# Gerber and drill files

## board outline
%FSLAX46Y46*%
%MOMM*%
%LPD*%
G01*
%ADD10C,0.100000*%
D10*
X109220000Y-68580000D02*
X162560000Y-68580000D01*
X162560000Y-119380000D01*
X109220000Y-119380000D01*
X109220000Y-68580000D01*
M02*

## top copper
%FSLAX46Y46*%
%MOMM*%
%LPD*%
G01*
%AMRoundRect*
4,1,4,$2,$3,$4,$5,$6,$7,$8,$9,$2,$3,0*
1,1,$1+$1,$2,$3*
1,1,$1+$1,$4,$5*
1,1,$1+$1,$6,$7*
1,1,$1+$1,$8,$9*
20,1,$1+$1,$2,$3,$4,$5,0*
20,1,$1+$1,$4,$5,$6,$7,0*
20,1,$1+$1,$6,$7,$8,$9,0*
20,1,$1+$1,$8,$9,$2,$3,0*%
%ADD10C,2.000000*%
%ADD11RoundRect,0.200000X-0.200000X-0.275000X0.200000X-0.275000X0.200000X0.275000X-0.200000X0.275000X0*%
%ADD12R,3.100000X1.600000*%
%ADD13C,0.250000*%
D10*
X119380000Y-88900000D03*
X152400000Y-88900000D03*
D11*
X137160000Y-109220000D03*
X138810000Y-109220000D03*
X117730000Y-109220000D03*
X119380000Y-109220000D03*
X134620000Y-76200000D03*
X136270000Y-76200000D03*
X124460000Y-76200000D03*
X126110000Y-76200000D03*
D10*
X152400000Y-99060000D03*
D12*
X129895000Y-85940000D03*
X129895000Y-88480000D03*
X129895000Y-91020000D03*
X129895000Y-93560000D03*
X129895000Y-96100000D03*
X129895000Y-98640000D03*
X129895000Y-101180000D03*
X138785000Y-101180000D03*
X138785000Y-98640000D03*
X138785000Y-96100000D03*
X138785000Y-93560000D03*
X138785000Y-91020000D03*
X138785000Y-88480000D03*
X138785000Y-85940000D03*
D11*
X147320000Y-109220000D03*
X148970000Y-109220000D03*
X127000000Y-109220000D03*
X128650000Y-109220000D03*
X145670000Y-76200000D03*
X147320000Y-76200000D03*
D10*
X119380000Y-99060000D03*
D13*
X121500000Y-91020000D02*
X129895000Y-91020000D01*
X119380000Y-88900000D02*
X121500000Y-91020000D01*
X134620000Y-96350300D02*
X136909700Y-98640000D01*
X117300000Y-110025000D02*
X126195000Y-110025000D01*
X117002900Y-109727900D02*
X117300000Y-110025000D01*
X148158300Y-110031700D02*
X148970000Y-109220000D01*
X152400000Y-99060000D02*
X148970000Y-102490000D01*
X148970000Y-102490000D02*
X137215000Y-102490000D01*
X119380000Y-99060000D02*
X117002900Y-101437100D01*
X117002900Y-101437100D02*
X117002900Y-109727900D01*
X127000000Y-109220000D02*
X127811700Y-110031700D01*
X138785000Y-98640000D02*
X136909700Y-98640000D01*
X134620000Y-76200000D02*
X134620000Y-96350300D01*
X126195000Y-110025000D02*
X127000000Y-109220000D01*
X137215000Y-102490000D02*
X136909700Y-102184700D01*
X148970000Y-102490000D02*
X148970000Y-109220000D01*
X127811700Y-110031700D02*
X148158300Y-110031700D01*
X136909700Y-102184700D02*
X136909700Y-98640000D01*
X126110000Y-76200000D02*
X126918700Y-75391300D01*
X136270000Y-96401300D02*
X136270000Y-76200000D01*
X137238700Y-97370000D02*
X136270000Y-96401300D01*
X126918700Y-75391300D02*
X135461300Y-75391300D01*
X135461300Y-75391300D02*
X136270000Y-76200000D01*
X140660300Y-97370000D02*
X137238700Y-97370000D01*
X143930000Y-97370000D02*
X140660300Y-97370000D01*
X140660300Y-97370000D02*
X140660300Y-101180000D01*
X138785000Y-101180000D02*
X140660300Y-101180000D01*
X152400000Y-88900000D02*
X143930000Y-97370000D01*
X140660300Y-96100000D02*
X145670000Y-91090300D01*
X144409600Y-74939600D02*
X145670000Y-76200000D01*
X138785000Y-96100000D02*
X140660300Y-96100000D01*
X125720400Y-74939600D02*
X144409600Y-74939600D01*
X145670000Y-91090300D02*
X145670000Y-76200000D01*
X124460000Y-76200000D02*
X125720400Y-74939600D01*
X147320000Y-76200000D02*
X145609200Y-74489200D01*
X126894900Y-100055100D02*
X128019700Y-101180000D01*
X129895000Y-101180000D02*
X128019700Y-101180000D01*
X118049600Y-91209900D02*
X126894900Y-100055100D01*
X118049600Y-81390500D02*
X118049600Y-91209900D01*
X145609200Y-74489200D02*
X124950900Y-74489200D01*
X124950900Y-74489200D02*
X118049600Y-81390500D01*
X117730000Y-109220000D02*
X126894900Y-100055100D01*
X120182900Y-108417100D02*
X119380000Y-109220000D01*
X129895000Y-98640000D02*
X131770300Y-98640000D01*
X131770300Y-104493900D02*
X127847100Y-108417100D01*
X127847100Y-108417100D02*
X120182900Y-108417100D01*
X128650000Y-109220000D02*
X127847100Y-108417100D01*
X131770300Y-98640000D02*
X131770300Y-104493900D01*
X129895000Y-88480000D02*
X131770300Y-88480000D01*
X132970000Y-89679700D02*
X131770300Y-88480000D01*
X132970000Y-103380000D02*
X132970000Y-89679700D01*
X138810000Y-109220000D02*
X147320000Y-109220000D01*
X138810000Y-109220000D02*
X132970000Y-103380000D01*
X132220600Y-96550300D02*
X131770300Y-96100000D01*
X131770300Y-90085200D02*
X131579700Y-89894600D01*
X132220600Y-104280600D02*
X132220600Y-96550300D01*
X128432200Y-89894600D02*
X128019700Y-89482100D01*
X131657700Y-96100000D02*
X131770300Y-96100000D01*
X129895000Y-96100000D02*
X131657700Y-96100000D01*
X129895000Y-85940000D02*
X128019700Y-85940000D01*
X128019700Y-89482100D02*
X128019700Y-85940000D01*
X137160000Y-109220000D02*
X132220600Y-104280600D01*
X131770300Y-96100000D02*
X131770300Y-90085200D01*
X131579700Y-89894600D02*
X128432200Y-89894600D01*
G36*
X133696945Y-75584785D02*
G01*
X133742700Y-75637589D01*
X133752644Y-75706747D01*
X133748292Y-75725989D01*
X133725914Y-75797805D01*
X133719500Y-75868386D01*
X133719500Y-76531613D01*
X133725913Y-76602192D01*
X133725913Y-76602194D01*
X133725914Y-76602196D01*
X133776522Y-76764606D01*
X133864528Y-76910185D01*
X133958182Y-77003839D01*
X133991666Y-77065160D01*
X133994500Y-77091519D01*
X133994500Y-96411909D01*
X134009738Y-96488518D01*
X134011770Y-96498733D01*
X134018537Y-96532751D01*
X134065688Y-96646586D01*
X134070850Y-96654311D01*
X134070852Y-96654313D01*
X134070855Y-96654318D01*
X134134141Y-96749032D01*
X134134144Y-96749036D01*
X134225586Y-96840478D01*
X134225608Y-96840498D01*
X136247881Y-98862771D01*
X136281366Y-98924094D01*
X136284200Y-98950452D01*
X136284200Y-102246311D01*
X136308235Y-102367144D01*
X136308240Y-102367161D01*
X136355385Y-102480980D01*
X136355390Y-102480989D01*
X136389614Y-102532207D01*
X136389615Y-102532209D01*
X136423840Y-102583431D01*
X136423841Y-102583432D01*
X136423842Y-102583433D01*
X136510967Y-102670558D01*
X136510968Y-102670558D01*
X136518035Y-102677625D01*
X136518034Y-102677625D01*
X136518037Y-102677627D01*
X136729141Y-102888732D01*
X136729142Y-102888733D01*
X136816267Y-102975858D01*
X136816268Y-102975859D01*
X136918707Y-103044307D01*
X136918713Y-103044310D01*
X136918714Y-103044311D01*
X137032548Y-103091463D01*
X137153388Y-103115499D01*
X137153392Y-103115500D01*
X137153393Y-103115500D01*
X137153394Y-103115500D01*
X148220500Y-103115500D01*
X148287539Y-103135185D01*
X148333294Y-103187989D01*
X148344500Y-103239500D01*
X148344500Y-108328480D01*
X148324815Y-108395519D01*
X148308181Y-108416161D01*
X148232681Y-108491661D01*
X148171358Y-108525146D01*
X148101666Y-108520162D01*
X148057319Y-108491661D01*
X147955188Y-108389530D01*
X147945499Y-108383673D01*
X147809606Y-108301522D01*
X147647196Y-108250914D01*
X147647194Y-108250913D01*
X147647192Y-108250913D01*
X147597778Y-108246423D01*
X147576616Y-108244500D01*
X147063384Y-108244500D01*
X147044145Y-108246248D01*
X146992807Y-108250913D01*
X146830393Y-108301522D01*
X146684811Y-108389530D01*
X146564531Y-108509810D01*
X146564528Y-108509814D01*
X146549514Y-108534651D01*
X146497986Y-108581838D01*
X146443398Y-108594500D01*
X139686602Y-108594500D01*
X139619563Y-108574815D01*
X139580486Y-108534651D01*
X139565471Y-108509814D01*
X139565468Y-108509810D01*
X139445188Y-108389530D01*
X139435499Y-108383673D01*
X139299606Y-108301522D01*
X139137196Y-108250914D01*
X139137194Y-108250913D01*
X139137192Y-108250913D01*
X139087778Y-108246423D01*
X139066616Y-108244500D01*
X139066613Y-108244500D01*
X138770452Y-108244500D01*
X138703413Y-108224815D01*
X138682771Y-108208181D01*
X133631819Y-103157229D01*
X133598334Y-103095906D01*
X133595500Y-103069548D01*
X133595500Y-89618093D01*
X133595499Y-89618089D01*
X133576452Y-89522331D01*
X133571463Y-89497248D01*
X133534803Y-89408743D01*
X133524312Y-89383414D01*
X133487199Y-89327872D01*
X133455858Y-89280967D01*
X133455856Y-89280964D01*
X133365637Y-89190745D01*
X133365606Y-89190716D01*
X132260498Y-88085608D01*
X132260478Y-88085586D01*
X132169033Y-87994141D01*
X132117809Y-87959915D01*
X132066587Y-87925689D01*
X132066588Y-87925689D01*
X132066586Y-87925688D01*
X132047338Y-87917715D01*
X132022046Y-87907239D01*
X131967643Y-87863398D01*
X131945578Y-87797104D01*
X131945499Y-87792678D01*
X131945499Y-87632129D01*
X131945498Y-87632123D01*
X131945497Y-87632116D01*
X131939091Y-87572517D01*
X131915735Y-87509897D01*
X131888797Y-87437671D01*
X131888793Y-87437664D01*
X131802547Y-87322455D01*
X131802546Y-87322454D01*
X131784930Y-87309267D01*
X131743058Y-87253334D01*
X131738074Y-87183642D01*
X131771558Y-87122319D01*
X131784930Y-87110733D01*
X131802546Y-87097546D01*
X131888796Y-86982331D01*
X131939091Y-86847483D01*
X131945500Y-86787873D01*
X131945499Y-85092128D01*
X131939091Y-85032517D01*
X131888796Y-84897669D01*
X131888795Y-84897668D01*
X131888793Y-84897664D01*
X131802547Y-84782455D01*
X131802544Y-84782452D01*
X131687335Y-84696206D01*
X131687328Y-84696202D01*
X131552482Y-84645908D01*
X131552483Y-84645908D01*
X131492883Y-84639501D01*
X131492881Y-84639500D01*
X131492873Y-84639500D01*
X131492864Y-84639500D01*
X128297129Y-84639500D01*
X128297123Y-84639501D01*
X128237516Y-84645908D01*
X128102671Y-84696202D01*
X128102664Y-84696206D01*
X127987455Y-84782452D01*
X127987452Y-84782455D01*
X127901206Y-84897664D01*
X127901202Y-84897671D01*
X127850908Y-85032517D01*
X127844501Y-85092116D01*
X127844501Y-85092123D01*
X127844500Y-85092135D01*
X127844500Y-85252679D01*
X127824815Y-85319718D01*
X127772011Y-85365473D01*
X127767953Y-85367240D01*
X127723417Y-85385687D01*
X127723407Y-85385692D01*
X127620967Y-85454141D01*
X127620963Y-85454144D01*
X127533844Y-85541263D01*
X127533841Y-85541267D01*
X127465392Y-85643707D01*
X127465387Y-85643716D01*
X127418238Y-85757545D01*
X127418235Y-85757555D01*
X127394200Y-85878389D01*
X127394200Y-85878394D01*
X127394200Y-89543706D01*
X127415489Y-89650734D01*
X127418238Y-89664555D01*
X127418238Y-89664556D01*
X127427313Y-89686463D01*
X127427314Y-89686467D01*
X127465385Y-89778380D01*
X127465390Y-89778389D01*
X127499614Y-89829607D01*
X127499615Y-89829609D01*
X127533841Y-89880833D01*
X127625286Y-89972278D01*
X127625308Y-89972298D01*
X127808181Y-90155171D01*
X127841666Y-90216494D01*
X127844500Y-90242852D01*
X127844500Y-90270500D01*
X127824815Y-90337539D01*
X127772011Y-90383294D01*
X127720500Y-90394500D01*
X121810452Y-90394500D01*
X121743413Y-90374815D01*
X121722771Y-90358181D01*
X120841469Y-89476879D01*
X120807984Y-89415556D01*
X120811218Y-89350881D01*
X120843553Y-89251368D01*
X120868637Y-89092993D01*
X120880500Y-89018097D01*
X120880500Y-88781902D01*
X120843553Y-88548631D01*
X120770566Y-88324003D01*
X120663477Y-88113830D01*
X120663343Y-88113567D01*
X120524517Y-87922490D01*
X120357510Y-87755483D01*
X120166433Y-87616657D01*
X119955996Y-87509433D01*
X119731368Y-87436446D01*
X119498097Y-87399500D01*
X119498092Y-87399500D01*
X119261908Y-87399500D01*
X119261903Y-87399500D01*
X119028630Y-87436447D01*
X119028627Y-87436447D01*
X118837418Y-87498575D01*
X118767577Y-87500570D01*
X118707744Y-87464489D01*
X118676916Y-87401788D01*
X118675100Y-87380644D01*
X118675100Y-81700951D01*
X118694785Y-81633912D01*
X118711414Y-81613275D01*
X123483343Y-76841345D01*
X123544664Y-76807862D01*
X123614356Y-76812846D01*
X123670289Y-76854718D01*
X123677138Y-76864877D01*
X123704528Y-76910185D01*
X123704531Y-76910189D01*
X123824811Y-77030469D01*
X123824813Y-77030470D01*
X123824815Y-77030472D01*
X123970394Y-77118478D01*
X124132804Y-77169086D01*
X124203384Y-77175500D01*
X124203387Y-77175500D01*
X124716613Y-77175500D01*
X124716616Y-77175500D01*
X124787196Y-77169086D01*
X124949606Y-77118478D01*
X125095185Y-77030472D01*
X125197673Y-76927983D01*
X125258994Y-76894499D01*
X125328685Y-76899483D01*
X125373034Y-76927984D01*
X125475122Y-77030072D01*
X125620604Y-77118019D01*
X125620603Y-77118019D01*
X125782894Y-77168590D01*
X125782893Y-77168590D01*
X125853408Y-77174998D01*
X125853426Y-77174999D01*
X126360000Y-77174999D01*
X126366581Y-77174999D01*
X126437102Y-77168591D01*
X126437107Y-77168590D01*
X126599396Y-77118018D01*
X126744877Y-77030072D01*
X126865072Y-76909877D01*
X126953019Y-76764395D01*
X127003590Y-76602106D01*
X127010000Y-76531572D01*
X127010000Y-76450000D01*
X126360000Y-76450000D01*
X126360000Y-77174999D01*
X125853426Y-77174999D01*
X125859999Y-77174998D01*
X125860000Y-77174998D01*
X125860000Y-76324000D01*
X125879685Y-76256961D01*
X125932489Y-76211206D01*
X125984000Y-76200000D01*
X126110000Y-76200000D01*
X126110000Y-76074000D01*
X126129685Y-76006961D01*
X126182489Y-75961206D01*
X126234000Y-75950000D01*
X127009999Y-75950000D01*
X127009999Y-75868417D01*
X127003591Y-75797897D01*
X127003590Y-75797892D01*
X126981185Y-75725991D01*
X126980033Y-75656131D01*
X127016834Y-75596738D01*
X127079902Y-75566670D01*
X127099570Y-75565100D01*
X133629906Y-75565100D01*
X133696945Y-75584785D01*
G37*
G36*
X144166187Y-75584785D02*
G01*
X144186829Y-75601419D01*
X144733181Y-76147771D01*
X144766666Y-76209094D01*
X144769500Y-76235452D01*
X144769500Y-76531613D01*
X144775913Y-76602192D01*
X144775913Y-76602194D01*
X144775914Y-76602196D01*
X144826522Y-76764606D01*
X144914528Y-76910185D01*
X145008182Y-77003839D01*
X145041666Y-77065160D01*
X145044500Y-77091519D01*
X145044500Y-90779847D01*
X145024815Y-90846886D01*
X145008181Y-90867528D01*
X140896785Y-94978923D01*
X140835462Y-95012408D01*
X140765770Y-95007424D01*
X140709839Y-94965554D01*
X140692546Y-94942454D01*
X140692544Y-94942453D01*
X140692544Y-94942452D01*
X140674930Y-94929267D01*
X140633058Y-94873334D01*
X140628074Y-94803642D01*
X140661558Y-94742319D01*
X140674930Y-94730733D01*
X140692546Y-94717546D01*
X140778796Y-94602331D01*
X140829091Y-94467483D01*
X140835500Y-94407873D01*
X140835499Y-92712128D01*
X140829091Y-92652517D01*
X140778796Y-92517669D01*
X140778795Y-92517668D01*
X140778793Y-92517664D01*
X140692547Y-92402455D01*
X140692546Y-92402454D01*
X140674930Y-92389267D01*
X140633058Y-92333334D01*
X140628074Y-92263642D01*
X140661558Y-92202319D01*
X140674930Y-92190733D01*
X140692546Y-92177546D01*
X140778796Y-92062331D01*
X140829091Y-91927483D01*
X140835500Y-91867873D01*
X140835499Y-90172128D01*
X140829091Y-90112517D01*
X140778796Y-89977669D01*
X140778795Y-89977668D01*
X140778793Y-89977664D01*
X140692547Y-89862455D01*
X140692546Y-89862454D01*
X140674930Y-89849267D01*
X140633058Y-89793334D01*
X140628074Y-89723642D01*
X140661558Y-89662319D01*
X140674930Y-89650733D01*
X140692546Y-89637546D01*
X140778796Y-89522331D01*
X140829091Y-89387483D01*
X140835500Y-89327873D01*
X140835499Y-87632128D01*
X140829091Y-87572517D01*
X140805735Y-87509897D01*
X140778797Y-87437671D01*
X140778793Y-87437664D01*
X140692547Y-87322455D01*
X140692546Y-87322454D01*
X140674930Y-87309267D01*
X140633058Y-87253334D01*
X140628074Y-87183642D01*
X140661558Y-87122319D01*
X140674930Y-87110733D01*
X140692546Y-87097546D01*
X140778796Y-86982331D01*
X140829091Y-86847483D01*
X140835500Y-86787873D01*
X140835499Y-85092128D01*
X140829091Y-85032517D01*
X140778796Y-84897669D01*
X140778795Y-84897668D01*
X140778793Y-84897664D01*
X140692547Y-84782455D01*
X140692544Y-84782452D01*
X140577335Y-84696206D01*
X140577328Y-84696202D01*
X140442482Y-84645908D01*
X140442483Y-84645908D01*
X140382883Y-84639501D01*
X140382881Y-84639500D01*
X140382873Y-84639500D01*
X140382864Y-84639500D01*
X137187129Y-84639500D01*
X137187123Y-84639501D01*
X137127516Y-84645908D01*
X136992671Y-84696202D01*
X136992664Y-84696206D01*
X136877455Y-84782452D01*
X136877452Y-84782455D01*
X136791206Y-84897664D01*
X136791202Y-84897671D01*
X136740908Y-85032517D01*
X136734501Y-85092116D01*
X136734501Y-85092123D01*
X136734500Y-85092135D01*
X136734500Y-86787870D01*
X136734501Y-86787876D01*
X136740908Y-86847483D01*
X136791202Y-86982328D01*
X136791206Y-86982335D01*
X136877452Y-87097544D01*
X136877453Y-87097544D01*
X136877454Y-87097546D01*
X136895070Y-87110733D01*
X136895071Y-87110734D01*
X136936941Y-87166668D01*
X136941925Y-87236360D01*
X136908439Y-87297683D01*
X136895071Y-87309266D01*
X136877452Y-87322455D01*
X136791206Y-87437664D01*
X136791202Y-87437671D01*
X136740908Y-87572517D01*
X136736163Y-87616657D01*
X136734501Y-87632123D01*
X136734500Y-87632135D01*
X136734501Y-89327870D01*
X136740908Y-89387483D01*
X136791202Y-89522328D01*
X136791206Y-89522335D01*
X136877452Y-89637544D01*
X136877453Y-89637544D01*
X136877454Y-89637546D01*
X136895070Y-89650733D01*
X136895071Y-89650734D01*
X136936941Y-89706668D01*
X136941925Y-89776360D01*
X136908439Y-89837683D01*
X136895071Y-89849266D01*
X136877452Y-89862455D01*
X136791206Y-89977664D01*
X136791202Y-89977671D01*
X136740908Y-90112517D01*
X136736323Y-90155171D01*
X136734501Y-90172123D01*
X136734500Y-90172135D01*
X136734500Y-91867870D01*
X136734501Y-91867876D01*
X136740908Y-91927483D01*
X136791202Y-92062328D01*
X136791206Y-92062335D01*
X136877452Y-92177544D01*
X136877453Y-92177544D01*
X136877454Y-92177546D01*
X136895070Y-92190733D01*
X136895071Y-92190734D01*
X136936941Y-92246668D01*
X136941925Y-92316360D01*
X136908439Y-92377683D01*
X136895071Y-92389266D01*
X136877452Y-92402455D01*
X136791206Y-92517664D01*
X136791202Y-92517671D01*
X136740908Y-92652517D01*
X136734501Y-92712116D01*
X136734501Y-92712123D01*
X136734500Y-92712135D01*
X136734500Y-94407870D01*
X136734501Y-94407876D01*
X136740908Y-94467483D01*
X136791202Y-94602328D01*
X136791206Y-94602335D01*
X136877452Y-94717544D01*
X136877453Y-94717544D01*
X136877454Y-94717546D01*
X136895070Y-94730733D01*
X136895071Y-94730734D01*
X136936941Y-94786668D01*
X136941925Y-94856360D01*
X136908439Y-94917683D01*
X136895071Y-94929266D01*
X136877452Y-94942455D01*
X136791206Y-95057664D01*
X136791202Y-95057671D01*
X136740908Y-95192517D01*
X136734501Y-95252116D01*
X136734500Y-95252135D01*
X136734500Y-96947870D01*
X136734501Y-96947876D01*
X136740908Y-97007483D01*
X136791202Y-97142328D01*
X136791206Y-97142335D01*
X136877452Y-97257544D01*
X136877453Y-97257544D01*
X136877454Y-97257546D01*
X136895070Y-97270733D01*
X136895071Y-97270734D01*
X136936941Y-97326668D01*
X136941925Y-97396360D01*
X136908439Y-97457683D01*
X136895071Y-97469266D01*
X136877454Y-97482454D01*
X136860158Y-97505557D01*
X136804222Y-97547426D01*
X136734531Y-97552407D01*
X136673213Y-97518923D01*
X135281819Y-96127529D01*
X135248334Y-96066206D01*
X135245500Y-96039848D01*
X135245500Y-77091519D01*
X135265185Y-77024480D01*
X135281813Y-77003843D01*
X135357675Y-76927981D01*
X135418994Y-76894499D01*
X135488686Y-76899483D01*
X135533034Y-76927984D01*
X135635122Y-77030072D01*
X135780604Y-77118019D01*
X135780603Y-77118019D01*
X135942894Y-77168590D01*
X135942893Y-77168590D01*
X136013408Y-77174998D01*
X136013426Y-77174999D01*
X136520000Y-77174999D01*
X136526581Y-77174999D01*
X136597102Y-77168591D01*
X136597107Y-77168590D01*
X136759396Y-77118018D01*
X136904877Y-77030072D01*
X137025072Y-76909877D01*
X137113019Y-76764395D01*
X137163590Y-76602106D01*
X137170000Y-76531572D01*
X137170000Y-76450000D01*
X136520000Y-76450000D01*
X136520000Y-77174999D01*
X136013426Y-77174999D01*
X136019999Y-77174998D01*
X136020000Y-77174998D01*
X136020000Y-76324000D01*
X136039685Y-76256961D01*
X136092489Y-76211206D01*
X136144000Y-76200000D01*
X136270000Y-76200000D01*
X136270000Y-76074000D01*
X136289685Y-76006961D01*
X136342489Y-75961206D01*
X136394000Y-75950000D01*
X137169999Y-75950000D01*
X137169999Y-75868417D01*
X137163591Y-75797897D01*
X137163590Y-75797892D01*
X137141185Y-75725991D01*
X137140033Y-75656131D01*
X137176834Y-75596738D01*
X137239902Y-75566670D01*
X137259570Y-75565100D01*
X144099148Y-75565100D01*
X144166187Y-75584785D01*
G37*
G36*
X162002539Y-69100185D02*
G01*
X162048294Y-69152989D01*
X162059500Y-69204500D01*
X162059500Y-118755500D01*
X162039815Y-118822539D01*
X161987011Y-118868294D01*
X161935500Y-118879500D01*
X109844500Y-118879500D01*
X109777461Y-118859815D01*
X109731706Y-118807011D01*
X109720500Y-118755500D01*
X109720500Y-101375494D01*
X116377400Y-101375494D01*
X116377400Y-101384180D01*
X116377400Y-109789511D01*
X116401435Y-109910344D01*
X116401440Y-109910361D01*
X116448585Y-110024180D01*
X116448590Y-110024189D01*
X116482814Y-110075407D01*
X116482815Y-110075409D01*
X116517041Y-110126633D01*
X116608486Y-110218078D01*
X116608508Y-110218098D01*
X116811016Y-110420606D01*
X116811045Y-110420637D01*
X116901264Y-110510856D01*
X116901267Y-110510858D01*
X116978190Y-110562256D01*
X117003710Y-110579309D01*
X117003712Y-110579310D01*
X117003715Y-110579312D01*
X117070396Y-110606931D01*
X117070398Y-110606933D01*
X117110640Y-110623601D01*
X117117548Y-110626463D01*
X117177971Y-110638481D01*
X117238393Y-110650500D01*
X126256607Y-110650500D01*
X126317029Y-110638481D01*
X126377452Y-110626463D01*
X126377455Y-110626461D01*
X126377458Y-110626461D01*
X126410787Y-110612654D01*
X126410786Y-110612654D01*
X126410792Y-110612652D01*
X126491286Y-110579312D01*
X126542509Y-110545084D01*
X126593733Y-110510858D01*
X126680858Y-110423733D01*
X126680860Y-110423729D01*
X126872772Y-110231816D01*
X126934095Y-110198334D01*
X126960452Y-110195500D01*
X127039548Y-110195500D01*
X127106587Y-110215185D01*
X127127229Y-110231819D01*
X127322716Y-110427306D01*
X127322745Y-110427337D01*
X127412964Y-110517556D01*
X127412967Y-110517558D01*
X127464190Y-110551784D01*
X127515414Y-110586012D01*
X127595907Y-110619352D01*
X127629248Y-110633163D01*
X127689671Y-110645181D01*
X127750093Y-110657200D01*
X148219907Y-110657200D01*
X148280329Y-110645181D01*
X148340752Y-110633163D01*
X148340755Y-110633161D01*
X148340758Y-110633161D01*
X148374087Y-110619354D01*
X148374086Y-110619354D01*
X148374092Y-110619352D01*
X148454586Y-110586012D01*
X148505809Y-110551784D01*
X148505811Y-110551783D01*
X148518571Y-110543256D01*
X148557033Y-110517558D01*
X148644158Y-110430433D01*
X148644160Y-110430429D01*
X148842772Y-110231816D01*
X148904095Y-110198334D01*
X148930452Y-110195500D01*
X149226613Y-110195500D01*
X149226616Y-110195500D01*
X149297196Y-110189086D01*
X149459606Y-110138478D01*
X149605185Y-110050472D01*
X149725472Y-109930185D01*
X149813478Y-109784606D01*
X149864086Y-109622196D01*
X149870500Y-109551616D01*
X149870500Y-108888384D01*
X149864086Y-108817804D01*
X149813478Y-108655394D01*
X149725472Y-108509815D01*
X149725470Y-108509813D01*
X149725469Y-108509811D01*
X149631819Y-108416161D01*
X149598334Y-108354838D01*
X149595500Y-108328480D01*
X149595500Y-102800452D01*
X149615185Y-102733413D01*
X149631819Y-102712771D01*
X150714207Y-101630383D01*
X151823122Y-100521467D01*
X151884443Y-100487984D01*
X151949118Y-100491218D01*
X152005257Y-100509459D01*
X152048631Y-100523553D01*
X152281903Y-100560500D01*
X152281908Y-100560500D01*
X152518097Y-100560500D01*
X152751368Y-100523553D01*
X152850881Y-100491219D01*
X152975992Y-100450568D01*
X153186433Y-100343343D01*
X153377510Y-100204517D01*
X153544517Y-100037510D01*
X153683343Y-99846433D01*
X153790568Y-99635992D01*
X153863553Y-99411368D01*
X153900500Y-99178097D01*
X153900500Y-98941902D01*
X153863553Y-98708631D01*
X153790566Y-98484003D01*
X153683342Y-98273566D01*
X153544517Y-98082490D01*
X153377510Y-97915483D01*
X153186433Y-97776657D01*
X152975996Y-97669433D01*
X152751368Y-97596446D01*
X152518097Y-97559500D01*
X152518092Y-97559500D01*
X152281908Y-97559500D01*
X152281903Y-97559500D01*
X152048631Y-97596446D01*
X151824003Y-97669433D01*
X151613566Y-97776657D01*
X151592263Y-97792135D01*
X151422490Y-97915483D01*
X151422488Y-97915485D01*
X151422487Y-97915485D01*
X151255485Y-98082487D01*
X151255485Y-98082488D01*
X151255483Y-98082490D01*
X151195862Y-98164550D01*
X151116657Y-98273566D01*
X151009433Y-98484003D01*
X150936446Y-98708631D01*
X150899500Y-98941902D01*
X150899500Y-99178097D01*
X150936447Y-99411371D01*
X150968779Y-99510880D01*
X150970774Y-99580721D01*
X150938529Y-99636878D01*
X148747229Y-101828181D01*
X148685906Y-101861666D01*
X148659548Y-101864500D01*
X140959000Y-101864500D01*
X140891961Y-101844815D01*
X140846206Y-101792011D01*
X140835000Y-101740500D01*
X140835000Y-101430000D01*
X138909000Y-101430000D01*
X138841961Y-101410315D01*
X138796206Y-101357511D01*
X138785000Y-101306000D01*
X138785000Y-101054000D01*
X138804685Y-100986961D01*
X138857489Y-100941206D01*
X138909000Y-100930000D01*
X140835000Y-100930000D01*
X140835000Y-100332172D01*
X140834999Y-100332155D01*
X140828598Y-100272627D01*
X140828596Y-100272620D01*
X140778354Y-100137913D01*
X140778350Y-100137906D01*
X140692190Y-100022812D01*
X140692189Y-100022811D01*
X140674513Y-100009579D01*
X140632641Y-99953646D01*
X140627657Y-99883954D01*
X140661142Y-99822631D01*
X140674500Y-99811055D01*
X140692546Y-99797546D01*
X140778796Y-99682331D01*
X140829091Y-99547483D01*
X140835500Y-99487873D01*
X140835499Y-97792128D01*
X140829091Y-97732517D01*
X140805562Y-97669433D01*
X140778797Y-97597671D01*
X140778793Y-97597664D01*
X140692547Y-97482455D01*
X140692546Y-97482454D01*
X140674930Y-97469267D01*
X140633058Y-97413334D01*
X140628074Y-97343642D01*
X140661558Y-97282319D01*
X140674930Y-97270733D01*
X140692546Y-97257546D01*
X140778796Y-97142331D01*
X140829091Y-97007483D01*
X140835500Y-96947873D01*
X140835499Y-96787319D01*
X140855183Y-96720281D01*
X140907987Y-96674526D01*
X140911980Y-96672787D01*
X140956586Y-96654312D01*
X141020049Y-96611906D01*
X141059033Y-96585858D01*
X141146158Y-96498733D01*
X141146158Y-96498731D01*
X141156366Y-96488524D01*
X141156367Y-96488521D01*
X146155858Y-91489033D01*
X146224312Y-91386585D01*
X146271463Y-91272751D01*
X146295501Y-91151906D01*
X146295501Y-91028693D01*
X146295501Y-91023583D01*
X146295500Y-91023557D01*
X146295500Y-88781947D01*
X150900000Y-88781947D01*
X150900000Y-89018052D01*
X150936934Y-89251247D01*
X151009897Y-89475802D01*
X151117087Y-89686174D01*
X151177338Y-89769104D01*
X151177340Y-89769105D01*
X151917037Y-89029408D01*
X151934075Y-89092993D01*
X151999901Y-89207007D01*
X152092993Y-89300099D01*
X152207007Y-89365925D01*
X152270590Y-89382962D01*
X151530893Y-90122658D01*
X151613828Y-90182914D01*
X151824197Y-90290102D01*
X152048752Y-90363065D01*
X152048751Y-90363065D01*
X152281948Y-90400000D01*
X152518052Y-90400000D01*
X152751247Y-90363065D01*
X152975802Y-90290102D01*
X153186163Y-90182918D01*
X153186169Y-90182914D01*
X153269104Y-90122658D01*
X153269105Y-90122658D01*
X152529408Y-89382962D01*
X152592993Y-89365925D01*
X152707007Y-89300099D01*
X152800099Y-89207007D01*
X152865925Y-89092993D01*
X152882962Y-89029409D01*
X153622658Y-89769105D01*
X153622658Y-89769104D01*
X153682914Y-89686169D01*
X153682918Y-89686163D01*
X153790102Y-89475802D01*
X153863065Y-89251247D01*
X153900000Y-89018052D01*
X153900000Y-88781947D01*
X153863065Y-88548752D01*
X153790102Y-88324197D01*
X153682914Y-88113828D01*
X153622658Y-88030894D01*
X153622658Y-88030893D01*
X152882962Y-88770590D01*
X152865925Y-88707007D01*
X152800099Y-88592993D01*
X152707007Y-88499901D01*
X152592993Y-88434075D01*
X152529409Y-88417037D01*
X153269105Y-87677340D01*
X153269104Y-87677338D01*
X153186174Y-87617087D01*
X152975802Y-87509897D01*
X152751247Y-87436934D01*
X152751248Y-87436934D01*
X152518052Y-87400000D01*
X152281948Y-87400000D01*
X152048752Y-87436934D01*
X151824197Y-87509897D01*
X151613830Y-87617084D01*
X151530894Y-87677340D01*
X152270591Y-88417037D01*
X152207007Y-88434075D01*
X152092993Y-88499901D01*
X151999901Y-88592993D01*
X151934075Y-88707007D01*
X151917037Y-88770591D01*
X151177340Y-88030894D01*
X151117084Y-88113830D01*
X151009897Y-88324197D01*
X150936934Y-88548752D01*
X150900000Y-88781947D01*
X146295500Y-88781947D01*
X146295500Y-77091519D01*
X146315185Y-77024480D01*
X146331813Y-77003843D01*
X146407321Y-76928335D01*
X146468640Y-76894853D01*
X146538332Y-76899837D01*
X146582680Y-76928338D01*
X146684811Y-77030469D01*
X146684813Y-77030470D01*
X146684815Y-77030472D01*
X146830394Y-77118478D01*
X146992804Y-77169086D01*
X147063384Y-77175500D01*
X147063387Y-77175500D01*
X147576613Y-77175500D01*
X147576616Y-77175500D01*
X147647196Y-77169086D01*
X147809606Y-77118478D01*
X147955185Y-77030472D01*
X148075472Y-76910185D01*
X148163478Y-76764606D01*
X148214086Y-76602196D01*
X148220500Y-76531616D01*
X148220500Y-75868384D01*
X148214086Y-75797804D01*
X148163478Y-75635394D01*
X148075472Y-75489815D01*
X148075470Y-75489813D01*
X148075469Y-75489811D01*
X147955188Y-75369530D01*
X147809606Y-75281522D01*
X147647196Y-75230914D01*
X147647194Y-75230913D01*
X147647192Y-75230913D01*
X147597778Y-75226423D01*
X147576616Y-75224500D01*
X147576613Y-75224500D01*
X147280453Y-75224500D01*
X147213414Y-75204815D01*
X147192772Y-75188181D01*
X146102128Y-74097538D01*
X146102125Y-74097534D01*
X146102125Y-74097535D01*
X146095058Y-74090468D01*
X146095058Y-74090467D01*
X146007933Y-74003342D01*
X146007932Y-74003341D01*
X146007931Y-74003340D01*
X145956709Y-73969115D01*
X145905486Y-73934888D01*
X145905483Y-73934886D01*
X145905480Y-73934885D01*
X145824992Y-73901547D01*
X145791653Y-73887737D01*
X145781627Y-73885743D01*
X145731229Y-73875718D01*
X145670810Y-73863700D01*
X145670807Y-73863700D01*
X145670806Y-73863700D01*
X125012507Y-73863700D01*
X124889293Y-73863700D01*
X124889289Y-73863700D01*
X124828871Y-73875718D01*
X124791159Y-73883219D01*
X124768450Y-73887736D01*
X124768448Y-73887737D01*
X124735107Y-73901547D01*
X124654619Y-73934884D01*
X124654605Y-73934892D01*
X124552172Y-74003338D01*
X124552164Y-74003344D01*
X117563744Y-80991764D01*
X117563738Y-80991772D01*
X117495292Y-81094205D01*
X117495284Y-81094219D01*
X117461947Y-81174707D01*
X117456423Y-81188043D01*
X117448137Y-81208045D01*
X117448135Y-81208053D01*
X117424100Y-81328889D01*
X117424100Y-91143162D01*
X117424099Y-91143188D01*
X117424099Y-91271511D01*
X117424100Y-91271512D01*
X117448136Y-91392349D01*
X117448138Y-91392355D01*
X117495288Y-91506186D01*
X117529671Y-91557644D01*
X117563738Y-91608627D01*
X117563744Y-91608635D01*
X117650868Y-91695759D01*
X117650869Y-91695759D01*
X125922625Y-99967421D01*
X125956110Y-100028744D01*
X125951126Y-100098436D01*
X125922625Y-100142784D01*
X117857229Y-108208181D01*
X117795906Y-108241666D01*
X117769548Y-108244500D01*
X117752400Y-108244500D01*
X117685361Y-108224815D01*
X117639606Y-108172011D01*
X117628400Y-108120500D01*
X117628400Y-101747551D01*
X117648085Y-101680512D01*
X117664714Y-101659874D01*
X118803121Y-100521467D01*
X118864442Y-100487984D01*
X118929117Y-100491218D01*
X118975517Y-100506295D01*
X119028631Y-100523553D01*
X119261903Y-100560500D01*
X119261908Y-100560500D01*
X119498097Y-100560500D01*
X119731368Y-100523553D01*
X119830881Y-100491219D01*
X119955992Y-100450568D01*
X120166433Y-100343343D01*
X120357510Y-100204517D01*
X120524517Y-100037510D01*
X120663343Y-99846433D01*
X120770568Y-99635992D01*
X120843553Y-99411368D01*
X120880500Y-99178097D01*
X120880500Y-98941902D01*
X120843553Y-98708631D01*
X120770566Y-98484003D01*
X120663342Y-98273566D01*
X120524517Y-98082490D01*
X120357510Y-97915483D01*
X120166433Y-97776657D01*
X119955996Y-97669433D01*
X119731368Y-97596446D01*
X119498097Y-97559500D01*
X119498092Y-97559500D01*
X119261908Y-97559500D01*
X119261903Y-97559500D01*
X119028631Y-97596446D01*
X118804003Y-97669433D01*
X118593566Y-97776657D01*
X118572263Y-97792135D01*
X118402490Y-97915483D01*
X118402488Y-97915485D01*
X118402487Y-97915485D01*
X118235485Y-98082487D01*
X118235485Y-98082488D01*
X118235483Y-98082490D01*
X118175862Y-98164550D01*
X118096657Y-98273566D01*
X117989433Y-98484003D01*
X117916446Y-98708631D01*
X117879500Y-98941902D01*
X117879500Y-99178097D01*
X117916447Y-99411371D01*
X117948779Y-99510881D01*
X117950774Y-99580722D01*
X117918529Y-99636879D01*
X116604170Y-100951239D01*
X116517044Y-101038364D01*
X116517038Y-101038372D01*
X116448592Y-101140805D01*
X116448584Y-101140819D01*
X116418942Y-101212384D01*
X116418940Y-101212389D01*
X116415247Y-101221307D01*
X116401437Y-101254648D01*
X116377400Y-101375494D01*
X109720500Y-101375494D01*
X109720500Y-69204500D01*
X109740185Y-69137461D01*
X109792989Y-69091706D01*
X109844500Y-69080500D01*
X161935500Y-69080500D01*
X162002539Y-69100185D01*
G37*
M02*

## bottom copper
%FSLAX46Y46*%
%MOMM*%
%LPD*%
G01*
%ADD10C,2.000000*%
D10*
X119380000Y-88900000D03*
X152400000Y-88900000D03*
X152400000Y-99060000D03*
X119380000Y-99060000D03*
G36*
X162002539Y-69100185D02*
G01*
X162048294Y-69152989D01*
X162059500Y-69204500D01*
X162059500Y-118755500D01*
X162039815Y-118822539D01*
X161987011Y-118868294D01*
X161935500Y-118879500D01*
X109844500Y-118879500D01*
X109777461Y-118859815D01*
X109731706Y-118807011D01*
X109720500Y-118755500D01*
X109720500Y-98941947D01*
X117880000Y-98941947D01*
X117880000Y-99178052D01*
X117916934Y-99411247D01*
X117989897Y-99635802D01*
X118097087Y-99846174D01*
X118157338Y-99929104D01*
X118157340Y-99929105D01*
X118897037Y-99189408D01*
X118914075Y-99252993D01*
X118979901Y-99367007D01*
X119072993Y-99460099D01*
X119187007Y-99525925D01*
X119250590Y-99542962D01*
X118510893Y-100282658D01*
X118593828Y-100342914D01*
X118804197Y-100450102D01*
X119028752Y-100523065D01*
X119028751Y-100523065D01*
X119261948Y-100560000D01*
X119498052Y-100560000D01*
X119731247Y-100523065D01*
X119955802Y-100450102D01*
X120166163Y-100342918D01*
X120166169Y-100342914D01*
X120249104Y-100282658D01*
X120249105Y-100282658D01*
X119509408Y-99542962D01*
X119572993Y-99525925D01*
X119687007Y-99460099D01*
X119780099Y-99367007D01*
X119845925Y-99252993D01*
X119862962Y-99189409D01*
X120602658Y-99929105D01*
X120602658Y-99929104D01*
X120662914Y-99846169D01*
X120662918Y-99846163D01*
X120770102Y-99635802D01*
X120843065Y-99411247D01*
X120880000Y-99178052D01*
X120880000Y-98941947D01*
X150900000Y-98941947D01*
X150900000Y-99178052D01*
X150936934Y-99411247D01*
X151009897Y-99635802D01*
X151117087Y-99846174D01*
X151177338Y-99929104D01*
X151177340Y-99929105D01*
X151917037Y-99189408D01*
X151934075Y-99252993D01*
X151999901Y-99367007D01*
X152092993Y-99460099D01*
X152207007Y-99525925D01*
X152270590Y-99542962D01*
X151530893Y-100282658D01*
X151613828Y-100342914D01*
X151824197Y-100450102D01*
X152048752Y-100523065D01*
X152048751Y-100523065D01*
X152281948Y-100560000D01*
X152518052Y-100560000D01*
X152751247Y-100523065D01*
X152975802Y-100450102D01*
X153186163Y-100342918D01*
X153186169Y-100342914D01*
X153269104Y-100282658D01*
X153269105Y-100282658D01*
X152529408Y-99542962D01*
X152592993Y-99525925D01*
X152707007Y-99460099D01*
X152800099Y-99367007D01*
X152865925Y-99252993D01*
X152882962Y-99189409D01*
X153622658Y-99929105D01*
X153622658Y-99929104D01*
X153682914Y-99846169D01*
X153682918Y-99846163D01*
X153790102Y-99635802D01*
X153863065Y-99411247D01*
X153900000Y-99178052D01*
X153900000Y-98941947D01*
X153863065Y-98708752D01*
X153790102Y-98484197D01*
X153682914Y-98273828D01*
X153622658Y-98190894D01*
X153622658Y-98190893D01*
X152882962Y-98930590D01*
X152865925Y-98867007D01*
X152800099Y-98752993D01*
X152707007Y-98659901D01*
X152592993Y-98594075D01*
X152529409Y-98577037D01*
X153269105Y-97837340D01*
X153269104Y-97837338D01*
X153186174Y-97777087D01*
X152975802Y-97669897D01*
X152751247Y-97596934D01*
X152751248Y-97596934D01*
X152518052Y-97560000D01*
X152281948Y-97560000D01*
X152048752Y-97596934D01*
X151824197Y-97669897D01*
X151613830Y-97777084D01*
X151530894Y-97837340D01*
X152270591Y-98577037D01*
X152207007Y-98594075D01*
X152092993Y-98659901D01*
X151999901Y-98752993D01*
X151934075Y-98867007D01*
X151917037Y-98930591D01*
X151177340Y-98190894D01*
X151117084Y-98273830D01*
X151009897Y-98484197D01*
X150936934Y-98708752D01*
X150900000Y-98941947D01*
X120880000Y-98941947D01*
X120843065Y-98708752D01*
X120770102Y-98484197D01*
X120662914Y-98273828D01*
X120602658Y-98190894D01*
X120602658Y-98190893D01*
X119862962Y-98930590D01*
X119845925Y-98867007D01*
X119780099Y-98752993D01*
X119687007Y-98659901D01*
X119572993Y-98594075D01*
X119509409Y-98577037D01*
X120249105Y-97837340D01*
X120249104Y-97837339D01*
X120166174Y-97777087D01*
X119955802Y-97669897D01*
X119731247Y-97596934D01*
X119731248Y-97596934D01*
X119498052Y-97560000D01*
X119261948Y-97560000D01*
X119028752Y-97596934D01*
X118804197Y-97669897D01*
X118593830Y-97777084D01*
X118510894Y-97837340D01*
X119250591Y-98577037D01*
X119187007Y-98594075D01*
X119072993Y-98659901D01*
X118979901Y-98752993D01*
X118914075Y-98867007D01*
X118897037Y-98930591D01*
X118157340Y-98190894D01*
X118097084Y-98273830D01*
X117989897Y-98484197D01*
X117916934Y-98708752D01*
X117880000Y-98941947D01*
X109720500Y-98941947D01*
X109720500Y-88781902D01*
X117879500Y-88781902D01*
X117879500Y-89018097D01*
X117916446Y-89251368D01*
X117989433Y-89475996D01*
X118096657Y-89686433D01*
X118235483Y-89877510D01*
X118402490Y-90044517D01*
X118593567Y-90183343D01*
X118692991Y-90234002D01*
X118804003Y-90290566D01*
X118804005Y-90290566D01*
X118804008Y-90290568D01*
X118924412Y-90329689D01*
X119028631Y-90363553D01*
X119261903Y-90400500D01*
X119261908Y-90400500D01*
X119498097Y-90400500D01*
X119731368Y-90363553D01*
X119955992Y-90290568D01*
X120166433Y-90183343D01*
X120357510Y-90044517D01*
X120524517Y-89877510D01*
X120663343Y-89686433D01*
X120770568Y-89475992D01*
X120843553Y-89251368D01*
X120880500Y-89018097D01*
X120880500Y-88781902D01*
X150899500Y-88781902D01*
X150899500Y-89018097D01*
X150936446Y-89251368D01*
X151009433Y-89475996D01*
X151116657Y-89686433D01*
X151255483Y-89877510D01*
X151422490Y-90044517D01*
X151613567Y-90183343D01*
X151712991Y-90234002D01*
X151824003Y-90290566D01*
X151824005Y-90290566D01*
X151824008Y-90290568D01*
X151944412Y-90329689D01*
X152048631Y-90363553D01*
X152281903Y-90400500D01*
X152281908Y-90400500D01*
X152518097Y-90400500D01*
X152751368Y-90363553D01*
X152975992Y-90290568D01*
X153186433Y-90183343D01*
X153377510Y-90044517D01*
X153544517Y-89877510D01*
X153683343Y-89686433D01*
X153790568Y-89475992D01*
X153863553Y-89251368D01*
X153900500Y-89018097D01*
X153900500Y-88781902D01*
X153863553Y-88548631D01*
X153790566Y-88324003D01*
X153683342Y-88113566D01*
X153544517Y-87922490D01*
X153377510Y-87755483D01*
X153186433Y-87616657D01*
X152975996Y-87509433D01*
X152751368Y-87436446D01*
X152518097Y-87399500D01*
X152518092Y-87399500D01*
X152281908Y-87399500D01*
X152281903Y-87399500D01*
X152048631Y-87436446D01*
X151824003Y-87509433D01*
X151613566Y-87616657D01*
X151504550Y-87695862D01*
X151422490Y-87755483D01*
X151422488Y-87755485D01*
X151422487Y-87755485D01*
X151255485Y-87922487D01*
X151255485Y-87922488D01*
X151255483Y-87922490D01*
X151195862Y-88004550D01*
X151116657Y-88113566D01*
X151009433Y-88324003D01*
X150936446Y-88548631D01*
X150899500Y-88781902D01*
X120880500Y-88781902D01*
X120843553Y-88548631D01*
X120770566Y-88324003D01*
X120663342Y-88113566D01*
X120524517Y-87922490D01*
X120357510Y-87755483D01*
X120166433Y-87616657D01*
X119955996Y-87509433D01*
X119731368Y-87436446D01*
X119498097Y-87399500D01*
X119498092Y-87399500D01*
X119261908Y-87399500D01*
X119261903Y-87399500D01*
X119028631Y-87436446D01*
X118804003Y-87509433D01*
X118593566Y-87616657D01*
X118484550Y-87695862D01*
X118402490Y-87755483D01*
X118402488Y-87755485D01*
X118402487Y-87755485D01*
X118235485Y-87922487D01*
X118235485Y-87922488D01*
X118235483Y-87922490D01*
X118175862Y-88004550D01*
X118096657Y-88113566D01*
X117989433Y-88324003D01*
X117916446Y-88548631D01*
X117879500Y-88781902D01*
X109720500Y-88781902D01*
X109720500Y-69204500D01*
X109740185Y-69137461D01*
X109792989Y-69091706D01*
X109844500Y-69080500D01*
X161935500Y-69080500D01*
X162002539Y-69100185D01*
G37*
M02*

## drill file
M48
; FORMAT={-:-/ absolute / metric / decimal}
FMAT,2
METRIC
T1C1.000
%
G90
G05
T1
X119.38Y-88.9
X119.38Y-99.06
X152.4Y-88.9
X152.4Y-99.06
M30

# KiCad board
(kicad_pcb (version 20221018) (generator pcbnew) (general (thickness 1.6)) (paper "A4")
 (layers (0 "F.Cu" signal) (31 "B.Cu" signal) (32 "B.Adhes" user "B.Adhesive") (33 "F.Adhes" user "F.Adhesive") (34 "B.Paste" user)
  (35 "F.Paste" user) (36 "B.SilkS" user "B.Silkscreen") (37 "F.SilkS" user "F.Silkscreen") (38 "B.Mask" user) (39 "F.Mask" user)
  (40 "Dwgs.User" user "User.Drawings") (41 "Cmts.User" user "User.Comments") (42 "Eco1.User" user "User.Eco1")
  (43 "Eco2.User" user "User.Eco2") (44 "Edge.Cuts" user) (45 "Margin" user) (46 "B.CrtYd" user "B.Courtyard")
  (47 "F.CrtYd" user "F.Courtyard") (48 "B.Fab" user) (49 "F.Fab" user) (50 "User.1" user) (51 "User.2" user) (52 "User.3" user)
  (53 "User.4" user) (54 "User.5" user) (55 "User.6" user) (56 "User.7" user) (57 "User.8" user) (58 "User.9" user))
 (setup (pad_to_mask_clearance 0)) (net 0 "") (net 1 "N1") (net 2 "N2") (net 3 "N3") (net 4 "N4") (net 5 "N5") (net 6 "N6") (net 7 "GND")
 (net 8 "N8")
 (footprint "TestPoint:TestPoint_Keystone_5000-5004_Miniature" (layer "F.Cu") (at 119.38 88.9)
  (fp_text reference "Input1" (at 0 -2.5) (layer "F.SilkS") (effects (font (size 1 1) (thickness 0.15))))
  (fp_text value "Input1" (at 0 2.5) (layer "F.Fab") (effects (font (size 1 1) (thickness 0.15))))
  (pad "1" thru_hole circle (at 0 0) (size 2 2) (drill 1) (layers "*.Cu" "*.Mask") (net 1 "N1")))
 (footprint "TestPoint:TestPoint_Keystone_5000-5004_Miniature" (layer "F.Cu") (at 152.4 88.9)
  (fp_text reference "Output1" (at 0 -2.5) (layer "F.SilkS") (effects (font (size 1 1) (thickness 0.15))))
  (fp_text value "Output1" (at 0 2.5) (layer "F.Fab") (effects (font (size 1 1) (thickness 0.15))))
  (pad "1" thru_hole circle (at 0 0) (size 2 2) (drill 1) (layers "*.Cu" "*.Mask") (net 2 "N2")))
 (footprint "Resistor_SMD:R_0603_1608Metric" (layer "F.Cu") (at 137.985 109.22)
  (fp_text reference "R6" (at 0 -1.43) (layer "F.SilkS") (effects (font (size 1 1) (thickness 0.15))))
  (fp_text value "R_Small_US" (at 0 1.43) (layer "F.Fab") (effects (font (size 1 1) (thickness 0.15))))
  (pad "1" smd roundrect (at -0.825 0) (size 0.8 0.95) (layers "F.Cu" "F.Paste" "F.Mask") (roundrect_rratio 0.25) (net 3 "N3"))
  (pad "2" smd roundrect (at 0.825 0) (size 0.8 0.95) (layers "F.Cu" "F.Paste" "F.Mask") (roundrect_rratio 0.25) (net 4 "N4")))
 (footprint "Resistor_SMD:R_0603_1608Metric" (layer "F.Cu") (at 118.555 109.22)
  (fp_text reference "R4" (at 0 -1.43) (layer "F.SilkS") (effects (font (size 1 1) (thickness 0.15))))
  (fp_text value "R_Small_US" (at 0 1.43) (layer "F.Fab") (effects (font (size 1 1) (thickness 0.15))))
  (pad "1" smd roundrect (at -0.825 0) (size 0.8 0.95) (layers "F.Cu" "F.Paste" "F.Mask") (roundrect_rratio 0.25) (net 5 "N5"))
  (pad "2" smd roundrect (at 0.825 0) (size 0.8 0.95) (layers "F.Cu" "F.Paste" "F.Mask") (roundrect_rratio 0.25) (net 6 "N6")))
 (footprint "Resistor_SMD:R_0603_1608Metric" (layer "F.Cu") (at 135.445 76.2)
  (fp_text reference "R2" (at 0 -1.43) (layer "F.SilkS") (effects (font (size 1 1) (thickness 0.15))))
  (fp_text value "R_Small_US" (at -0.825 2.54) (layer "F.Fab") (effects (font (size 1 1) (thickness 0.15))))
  (pad "1" smd roundrect (at -0.825 0) (size 0.8 0.95) (layers "F.Cu" "F.Paste" "F.Mask") (roundrect_rratio 0.25) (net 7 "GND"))
  (pad "2" smd roundrect (at 0.825 0) (size 0.8 0.95) (layers "F.Cu" "F.Paste" "F.Mask") (roundrect_rratio 0.25) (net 2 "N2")))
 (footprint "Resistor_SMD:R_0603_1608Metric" (layer "F.Cu") (at 125.285 76.2)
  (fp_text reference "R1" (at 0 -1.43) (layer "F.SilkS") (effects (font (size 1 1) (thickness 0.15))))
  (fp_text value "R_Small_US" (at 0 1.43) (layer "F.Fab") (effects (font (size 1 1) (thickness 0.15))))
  (pad "1" smd roundrect (at -0.825 0) (size 0.8 0.95) (layers "F.Cu" "F.Paste" "F.Mask") (roundrect_rratio 0.25) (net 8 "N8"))
  (pad "2" smd roundrect (at 0.825 0) (size 0.8 0.95) (layers "F.Cu" "F.Paste" "F.Mask") (roundrect_rratio 0.25) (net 2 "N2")))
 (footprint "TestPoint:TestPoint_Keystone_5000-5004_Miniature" (layer "F.Cu") (at 152.4 99.06)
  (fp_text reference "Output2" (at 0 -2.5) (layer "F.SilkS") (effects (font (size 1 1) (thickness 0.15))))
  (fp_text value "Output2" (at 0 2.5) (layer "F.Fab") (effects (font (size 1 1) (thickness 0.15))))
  (pad "1" thru_hole circle (at 0 0) (size 2 2) (drill 1) (layers "*.Cu" "*.Mask") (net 7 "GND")))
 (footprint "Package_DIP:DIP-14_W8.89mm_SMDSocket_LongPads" (layer "F.Cu") (at 134.34 93.56)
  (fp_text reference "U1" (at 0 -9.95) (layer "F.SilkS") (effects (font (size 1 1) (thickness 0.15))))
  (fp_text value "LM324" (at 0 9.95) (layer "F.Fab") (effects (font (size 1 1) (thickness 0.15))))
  (pad "1" smd rect (at -4.445 -7.62) (size 3.1 1.6) (layers "F.Cu" "F.Paste" "F.Mask") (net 3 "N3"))
  (pad "2" smd rect (at -4.445 -5.08) (size 3.1 1.6) (layers "F.Cu" "F.Paste" "F.Mask") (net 4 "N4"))
  (pad "3" smd rect (at -4.445 -2.54) (size 3.1 1.6) (layers "F.Cu" "F.Paste" "F.Mask") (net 1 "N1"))
  (pad "4" smd rect (at -4.445 0) (size 3.1 1.6) (layers "F.Cu" "F.Paste" "F.Mask"))
  (pad "5" smd rect (at -4.445 2.54) (size 3.1 1.6) (layers "F.Cu" "F.Paste" "F.Mask") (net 3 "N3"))
  (pad "6" smd rect (at -4.445 5.08) (size 3.1 1.6) (layers "F.Cu" "F.Paste" "F.Mask") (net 6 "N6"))
  (pad "7" smd rect (at -4.445 7.62) (size 3.1 1.6) (layers "F.Cu" "F.Paste" "F.Mask") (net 5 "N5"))
  (pad "8" smd rect (at 4.445 7.62) (size 3.1 1.6) (layers "F.Cu" "F.Paste" "F.Mask") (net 2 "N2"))
  (pad "9" smd rect (at 4.445 5.08) (size 3.1 1.6) (layers "F.Cu" "F.Paste" "F.Mask") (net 7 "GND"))
  (pad "10" smd rect (at 4.445 2.54) (size 3.1 1.6) (layers "F.Cu" "F.Paste" "F.Mask") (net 8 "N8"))
  (pad "11" smd rect (at 4.445 0) (size 3.1 1.6) (layers "F.Cu" "F.Paste" "F.Mask"))
  (pad "12" smd rect (at 4.445 -2.54) (size 3.1 1.6) (layers "F.Cu" "F.Paste" "F.Mask"))
  (pad "13" smd rect (at 4.445 -5.08) (size 3.1 1.6) (layers "F.Cu" "F.Paste" "F.Mask"))
  (pad "14" smd rect (at 4.445 -7.62) (size 3.1 1.6) (layers "F.Cu" "F.Paste" "F.Mask")))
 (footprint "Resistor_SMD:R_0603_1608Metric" (layer "F.Cu") (at 148.145 109.22)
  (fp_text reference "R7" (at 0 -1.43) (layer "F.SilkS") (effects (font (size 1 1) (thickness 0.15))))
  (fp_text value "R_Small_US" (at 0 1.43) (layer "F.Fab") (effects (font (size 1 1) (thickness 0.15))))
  (pad "1" smd roundrect (at -0.825 0) (size 0.8 0.95) (layers "F.Cu" "F.Paste" "F.Mask") (roundrect_rratio 0.25) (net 4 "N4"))
  (pad "2" smd roundrect (at 0.825 0) (size 0.8 0.95) (layers "F.Cu" "F.Paste" "F.Mask") (roundrect_rratio 0.25) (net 7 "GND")))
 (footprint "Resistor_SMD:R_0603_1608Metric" (layer "F.Cu") (at 127.825 109.22)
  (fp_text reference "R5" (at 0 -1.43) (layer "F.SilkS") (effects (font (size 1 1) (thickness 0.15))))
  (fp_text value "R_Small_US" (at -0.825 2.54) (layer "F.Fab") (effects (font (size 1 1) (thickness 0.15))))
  (pad "1" smd roundrect (at -0.825 0) (size 0.8 0.95) (layers "F.Cu" "F.Paste" "F.Mask") (roundrect_rratio 0.25) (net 7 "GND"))
  (pad "2" smd roundrect (at 0.825 0) (size 0.8 0.95) (layers "F.Cu" "F.Paste" "F.Mask") (roundrect_rratio 0.25) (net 6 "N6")))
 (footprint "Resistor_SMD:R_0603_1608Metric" (layer "F.Cu") (at 146.495 76.2)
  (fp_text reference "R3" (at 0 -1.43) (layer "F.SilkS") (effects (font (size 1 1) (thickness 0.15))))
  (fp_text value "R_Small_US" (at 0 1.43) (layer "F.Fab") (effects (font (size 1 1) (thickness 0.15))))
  (pad "1" smd roundrect (at -0.825 0) (size 0.8 0.95) (layers "F.Cu" "F.Paste" "F.Mask") (roundrect_rratio 0.25) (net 8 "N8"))
  (pad "2" smd roundrect (at 0.825 0) (size 0.8 0.95) (layers "F.Cu" "F.Paste" "F.Mask") (roundrect_rratio 0.25) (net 5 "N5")))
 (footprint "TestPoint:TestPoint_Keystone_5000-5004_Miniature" (layer "F.Cu") (at 119.38 99.06)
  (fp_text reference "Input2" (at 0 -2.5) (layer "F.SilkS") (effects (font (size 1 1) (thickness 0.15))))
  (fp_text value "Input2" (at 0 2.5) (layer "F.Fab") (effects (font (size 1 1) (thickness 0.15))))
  (pad "1" thru_hole circle (at 0 0) (size 2 2) (drill 1) (layers "*.Cu" "*.Mask") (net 7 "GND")))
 (gr_rect (start 109.22 68.58) (end 162.56 119.38) (stroke (width 0.1) (type default)) (fill none) (layer "Edge.Cuts"))
 (segment (start 121.5 91.02) (end 129.895 91.02) (width 0.25) (layer "F.Cu") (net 1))
 (segment (start 119.38 88.9) (end 121.5 91.02) (width 0.25) (layer "F.Cu") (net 1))
 (segment (start 134.62 96.3503) (end 136.9097 98.64) (width 0.25) (layer "F.Cu") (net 7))
 (segment (start 117.3 110.025) (end 126.195 110.025) (width 0.25) (layer "F.Cu") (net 7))
 (segment (start 117.0029 109.7279) (end 117.3 110.025) (width 0.25) (layer "F.Cu") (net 7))
 (segment (start 148.1583 110.0317) (end 148.97 109.22) (width 0.25) (layer "F.Cu") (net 7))
 (segment (start 152.4 99.06) (end 148.97 102.49) (width 0.25) (layer "F.Cu") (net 7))
 (segment (start 148.97 102.49) (end 137.215 102.49) (width 0.25) (layer "F.Cu") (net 7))
 (segment (start 119.38 99.06) (end 117.0029 101.4371) (width 0.25) (layer "F.Cu") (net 7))
 (segment (start 117.0029 101.4371) (end 117.0029 109.7279) (width 0.25) (layer "F.Cu") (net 7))
 (segment (start 127 109.22) (end 127.8117 110.0317) (width 0.25) (layer "F.Cu") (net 7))
 (segment (start 138.785 98.64) (end 136.9097 98.64) (width 0.25) (layer "F.Cu") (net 7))
 (segment (start 134.62 76.2) (end 134.62 96.3503) (width 0.25) (layer "F.Cu") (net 7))
 (segment (start 126.195 110.025) (end 127 109.22) (width 0.25) (layer "F.Cu") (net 7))
 (segment (start 137.215 102.49) (end 136.9097 102.1847) (width 0.25) (layer "F.Cu") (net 7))
 (segment (start 148.97 102.49) (end 148.97 109.22) (width 0.25) (layer "F.Cu") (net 7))
 (segment (start 127.8117 110.0317) (end 148.1583 110.0317) (width 0.25) (layer "F.Cu") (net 7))
 (segment (start 136.9097 102.1847) (end 136.9097 98.64) (width 0.25) (layer "F.Cu") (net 7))
 (segment (start 126.11 76.2) (end 126.9187 75.3913) (width 0.25) (layer "F.Cu") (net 2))
 (segment (start 136.27 96.4013) (end 136.27 76.2) (width 0.25) (layer "F.Cu") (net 2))
 (segment (start 137.2387 97.37) (end 136.27 96.4013) (width 0.25) (layer "F.Cu") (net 2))
 (segment (start 126.9187 75.3913) (end 135.4613 75.3913) (width 0.25) (layer "F.Cu") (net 2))
 (segment (start 135.4613 75.3913) (end 136.27 76.2) (width 0.25) (layer "F.Cu") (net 2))
 (segment (start 140.6603 97.37) (end 137.2387 97.37) (width 0.25) (layer "F.Cu") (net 2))
 (segment (start 143.93 97.37) (end 140.6603 97.37) (width 0.25) (layer "F.Cu") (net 2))
 (segment (start 140.6603 97.37) (end 140.6603 101.18) (width 0.25) (layer "F.Cu") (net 2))
 (segment (start 138.785 101.18) (end 140.6603 101.18) (width 0.25) (layer "F.Cu") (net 2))
 (segment (start 152.4 88.9) (end 143.93 97.37) (width 0.25) (layer "F.Cu") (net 2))
 (segment (start 140.6603 96.1) (end 145.67 91.0903) (width 0.25) (layer "F.Cu") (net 8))
 (segment (start 144.4096 74.9396) (end 145.67 76.2) (width 0.25) (layer "F.Cu") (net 8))
 (segment (start 138.785 96.1) (end 140.6603 96.1) (width 0.25) (layer "F.Cu") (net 8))
 (segment (start 125.7204 74.9396) (end 144.4096 74.9396) (width 0.25) (layer "F.Cu") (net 8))
 (segment (start 145.67 91.0903) (end 145.67 76.2) (width 0.25) (layer "F.Cu") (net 8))
 (segment (start 124.46 76.2) (end 125.7204 74.9396) (width 0.25) (layer "F.Cu") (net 8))
 (segment (start 147.32 76.2) (end 145.6092 74.4892) (width 0.25) (layer "F.Cu") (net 5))
 (segment (start 126.8949 100.0551) (end 128.0197 101.18) (width 0.25) (layer "F.Cu") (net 5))
 (segment (start 129.895 101.18) (end 128.0197 101.18) (width 0.25) (layer "F.Cu") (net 5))
 (segment (start 118.0496 91.2099) (end 126.8949 100.0551) (width 0.25) (layer "F.Cu") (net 5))
 (segment (start 118.0496 81.3905) (end 118.0496 91.2099) (width 0.25) (layer "F.Cu") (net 5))
 (segment (start 145.6092 74.4892) (end 124.9509 74.4892) (width 0.25) (layer "F.Cu") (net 5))
 (segment (start 124.9509 74.4892) (end 118.0496 81.3905) (width 0.25) (layer "F.Cu") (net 5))
 (segment (start 117.73 109.22) (end 126.8949 100.0551) (width 0.25) (layer "F.Cu") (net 5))
 (segment (start 120.1829 108.4171) (end 119.38 109.22) (width 0.25) (layer "F.Cu") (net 6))
 (segment (start 129.895 98.64) (end 131.7703 98.64) (width 0.25) (layer "F.Cu") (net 6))
 (segment (start 131.7703 104.4939) (end 127.8471 108.4171) (width 0.25) (layer "F.Cu") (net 6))
 (segment (start 127.8471 108.4171) (end 120.1829 108.4171) (width 0.25) (layer "F.Cu") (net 6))
 (segment (start 128.65 109.22) (end 127.8471 108.4171) (width 0.25) (layer "F.Cu") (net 6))
 (segment (start 131.7703 98.64) (end 131.7703 104.4939) (width 0.25) (layer "F.Cu") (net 6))
 (segment (start 129.895 88.48) (end 131.7703 88.48) (width 0.25) (layer "F.Cu") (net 4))
 (segment (start 132.97 89.6797) (end 131.7703 88.48) (width 0.25) (layer "F.Cu") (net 4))
 (segment (start 132.97 103.38) (end 132.97 89.6797) (width 0.25) (layer "F.Cu") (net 4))
 (segment (start 138.81 109.22) (end 147.32 109.22) (width 0.25) (layer "F.Cu") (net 4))
 (segment (start 138.81 109.22) (end 132.97 103.38) (width 0.25) (layer "F.Cu") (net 4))
 (segment (start 132.2206 96.5503) (end 131.7703 96.1) (width 0.25) (layer "F.Cu") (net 3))
 (segment (start 131.7703 90.0852) (end 131.5797 89.8946) (width 0.25) (layer "F.Cu") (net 3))
 (segment (start 132.2206 104.2806) (end 132.2206 96.5503) (width 0.25) (layer "F.Cu") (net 3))
 (segment (start 128.4322 89.8946) (end 128.0197 89.4821) (width 0.25) (layer "F.Cu") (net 3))
 (segment (start 131.6577 96.1) (end 131.7703 96.1) (width 0.25) (layer "F.Cu") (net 3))
 (segment (start 129.895 96.1) (end 131.6577 96.1) (width 0.25) (layer "F.Cu") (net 3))
 (segment (start 129.895 85.94) (end 128.0197 85.94) (width 0.25) (layer "F.Cu") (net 3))
 (segment (start 128.0197 89.4821) (end 128.0197 85.94) (width 0.25) (layer "F.Cu") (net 3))
 (segment (start 137.16 109.22) (end 132.2206 104.2806) (width 0.25) (layer "F.Cu") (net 3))
 (segment (start 131.7703 96.1) (end 131.7703 90.0852) (width 0.25) (layer "F.Cu") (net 3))
 (segment (start 131.5797 89.8946) (end 128.4322 89.8946) (width 0.25) (layer "F.Cu") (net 3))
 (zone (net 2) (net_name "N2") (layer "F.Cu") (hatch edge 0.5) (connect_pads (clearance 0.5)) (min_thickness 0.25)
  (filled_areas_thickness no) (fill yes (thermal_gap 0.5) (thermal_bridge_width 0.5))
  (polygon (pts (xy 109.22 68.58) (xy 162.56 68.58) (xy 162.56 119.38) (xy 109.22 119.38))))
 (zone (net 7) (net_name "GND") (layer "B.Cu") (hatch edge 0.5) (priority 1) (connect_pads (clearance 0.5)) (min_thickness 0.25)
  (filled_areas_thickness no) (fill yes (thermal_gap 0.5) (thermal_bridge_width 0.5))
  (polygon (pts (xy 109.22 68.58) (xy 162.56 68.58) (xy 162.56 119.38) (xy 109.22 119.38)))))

